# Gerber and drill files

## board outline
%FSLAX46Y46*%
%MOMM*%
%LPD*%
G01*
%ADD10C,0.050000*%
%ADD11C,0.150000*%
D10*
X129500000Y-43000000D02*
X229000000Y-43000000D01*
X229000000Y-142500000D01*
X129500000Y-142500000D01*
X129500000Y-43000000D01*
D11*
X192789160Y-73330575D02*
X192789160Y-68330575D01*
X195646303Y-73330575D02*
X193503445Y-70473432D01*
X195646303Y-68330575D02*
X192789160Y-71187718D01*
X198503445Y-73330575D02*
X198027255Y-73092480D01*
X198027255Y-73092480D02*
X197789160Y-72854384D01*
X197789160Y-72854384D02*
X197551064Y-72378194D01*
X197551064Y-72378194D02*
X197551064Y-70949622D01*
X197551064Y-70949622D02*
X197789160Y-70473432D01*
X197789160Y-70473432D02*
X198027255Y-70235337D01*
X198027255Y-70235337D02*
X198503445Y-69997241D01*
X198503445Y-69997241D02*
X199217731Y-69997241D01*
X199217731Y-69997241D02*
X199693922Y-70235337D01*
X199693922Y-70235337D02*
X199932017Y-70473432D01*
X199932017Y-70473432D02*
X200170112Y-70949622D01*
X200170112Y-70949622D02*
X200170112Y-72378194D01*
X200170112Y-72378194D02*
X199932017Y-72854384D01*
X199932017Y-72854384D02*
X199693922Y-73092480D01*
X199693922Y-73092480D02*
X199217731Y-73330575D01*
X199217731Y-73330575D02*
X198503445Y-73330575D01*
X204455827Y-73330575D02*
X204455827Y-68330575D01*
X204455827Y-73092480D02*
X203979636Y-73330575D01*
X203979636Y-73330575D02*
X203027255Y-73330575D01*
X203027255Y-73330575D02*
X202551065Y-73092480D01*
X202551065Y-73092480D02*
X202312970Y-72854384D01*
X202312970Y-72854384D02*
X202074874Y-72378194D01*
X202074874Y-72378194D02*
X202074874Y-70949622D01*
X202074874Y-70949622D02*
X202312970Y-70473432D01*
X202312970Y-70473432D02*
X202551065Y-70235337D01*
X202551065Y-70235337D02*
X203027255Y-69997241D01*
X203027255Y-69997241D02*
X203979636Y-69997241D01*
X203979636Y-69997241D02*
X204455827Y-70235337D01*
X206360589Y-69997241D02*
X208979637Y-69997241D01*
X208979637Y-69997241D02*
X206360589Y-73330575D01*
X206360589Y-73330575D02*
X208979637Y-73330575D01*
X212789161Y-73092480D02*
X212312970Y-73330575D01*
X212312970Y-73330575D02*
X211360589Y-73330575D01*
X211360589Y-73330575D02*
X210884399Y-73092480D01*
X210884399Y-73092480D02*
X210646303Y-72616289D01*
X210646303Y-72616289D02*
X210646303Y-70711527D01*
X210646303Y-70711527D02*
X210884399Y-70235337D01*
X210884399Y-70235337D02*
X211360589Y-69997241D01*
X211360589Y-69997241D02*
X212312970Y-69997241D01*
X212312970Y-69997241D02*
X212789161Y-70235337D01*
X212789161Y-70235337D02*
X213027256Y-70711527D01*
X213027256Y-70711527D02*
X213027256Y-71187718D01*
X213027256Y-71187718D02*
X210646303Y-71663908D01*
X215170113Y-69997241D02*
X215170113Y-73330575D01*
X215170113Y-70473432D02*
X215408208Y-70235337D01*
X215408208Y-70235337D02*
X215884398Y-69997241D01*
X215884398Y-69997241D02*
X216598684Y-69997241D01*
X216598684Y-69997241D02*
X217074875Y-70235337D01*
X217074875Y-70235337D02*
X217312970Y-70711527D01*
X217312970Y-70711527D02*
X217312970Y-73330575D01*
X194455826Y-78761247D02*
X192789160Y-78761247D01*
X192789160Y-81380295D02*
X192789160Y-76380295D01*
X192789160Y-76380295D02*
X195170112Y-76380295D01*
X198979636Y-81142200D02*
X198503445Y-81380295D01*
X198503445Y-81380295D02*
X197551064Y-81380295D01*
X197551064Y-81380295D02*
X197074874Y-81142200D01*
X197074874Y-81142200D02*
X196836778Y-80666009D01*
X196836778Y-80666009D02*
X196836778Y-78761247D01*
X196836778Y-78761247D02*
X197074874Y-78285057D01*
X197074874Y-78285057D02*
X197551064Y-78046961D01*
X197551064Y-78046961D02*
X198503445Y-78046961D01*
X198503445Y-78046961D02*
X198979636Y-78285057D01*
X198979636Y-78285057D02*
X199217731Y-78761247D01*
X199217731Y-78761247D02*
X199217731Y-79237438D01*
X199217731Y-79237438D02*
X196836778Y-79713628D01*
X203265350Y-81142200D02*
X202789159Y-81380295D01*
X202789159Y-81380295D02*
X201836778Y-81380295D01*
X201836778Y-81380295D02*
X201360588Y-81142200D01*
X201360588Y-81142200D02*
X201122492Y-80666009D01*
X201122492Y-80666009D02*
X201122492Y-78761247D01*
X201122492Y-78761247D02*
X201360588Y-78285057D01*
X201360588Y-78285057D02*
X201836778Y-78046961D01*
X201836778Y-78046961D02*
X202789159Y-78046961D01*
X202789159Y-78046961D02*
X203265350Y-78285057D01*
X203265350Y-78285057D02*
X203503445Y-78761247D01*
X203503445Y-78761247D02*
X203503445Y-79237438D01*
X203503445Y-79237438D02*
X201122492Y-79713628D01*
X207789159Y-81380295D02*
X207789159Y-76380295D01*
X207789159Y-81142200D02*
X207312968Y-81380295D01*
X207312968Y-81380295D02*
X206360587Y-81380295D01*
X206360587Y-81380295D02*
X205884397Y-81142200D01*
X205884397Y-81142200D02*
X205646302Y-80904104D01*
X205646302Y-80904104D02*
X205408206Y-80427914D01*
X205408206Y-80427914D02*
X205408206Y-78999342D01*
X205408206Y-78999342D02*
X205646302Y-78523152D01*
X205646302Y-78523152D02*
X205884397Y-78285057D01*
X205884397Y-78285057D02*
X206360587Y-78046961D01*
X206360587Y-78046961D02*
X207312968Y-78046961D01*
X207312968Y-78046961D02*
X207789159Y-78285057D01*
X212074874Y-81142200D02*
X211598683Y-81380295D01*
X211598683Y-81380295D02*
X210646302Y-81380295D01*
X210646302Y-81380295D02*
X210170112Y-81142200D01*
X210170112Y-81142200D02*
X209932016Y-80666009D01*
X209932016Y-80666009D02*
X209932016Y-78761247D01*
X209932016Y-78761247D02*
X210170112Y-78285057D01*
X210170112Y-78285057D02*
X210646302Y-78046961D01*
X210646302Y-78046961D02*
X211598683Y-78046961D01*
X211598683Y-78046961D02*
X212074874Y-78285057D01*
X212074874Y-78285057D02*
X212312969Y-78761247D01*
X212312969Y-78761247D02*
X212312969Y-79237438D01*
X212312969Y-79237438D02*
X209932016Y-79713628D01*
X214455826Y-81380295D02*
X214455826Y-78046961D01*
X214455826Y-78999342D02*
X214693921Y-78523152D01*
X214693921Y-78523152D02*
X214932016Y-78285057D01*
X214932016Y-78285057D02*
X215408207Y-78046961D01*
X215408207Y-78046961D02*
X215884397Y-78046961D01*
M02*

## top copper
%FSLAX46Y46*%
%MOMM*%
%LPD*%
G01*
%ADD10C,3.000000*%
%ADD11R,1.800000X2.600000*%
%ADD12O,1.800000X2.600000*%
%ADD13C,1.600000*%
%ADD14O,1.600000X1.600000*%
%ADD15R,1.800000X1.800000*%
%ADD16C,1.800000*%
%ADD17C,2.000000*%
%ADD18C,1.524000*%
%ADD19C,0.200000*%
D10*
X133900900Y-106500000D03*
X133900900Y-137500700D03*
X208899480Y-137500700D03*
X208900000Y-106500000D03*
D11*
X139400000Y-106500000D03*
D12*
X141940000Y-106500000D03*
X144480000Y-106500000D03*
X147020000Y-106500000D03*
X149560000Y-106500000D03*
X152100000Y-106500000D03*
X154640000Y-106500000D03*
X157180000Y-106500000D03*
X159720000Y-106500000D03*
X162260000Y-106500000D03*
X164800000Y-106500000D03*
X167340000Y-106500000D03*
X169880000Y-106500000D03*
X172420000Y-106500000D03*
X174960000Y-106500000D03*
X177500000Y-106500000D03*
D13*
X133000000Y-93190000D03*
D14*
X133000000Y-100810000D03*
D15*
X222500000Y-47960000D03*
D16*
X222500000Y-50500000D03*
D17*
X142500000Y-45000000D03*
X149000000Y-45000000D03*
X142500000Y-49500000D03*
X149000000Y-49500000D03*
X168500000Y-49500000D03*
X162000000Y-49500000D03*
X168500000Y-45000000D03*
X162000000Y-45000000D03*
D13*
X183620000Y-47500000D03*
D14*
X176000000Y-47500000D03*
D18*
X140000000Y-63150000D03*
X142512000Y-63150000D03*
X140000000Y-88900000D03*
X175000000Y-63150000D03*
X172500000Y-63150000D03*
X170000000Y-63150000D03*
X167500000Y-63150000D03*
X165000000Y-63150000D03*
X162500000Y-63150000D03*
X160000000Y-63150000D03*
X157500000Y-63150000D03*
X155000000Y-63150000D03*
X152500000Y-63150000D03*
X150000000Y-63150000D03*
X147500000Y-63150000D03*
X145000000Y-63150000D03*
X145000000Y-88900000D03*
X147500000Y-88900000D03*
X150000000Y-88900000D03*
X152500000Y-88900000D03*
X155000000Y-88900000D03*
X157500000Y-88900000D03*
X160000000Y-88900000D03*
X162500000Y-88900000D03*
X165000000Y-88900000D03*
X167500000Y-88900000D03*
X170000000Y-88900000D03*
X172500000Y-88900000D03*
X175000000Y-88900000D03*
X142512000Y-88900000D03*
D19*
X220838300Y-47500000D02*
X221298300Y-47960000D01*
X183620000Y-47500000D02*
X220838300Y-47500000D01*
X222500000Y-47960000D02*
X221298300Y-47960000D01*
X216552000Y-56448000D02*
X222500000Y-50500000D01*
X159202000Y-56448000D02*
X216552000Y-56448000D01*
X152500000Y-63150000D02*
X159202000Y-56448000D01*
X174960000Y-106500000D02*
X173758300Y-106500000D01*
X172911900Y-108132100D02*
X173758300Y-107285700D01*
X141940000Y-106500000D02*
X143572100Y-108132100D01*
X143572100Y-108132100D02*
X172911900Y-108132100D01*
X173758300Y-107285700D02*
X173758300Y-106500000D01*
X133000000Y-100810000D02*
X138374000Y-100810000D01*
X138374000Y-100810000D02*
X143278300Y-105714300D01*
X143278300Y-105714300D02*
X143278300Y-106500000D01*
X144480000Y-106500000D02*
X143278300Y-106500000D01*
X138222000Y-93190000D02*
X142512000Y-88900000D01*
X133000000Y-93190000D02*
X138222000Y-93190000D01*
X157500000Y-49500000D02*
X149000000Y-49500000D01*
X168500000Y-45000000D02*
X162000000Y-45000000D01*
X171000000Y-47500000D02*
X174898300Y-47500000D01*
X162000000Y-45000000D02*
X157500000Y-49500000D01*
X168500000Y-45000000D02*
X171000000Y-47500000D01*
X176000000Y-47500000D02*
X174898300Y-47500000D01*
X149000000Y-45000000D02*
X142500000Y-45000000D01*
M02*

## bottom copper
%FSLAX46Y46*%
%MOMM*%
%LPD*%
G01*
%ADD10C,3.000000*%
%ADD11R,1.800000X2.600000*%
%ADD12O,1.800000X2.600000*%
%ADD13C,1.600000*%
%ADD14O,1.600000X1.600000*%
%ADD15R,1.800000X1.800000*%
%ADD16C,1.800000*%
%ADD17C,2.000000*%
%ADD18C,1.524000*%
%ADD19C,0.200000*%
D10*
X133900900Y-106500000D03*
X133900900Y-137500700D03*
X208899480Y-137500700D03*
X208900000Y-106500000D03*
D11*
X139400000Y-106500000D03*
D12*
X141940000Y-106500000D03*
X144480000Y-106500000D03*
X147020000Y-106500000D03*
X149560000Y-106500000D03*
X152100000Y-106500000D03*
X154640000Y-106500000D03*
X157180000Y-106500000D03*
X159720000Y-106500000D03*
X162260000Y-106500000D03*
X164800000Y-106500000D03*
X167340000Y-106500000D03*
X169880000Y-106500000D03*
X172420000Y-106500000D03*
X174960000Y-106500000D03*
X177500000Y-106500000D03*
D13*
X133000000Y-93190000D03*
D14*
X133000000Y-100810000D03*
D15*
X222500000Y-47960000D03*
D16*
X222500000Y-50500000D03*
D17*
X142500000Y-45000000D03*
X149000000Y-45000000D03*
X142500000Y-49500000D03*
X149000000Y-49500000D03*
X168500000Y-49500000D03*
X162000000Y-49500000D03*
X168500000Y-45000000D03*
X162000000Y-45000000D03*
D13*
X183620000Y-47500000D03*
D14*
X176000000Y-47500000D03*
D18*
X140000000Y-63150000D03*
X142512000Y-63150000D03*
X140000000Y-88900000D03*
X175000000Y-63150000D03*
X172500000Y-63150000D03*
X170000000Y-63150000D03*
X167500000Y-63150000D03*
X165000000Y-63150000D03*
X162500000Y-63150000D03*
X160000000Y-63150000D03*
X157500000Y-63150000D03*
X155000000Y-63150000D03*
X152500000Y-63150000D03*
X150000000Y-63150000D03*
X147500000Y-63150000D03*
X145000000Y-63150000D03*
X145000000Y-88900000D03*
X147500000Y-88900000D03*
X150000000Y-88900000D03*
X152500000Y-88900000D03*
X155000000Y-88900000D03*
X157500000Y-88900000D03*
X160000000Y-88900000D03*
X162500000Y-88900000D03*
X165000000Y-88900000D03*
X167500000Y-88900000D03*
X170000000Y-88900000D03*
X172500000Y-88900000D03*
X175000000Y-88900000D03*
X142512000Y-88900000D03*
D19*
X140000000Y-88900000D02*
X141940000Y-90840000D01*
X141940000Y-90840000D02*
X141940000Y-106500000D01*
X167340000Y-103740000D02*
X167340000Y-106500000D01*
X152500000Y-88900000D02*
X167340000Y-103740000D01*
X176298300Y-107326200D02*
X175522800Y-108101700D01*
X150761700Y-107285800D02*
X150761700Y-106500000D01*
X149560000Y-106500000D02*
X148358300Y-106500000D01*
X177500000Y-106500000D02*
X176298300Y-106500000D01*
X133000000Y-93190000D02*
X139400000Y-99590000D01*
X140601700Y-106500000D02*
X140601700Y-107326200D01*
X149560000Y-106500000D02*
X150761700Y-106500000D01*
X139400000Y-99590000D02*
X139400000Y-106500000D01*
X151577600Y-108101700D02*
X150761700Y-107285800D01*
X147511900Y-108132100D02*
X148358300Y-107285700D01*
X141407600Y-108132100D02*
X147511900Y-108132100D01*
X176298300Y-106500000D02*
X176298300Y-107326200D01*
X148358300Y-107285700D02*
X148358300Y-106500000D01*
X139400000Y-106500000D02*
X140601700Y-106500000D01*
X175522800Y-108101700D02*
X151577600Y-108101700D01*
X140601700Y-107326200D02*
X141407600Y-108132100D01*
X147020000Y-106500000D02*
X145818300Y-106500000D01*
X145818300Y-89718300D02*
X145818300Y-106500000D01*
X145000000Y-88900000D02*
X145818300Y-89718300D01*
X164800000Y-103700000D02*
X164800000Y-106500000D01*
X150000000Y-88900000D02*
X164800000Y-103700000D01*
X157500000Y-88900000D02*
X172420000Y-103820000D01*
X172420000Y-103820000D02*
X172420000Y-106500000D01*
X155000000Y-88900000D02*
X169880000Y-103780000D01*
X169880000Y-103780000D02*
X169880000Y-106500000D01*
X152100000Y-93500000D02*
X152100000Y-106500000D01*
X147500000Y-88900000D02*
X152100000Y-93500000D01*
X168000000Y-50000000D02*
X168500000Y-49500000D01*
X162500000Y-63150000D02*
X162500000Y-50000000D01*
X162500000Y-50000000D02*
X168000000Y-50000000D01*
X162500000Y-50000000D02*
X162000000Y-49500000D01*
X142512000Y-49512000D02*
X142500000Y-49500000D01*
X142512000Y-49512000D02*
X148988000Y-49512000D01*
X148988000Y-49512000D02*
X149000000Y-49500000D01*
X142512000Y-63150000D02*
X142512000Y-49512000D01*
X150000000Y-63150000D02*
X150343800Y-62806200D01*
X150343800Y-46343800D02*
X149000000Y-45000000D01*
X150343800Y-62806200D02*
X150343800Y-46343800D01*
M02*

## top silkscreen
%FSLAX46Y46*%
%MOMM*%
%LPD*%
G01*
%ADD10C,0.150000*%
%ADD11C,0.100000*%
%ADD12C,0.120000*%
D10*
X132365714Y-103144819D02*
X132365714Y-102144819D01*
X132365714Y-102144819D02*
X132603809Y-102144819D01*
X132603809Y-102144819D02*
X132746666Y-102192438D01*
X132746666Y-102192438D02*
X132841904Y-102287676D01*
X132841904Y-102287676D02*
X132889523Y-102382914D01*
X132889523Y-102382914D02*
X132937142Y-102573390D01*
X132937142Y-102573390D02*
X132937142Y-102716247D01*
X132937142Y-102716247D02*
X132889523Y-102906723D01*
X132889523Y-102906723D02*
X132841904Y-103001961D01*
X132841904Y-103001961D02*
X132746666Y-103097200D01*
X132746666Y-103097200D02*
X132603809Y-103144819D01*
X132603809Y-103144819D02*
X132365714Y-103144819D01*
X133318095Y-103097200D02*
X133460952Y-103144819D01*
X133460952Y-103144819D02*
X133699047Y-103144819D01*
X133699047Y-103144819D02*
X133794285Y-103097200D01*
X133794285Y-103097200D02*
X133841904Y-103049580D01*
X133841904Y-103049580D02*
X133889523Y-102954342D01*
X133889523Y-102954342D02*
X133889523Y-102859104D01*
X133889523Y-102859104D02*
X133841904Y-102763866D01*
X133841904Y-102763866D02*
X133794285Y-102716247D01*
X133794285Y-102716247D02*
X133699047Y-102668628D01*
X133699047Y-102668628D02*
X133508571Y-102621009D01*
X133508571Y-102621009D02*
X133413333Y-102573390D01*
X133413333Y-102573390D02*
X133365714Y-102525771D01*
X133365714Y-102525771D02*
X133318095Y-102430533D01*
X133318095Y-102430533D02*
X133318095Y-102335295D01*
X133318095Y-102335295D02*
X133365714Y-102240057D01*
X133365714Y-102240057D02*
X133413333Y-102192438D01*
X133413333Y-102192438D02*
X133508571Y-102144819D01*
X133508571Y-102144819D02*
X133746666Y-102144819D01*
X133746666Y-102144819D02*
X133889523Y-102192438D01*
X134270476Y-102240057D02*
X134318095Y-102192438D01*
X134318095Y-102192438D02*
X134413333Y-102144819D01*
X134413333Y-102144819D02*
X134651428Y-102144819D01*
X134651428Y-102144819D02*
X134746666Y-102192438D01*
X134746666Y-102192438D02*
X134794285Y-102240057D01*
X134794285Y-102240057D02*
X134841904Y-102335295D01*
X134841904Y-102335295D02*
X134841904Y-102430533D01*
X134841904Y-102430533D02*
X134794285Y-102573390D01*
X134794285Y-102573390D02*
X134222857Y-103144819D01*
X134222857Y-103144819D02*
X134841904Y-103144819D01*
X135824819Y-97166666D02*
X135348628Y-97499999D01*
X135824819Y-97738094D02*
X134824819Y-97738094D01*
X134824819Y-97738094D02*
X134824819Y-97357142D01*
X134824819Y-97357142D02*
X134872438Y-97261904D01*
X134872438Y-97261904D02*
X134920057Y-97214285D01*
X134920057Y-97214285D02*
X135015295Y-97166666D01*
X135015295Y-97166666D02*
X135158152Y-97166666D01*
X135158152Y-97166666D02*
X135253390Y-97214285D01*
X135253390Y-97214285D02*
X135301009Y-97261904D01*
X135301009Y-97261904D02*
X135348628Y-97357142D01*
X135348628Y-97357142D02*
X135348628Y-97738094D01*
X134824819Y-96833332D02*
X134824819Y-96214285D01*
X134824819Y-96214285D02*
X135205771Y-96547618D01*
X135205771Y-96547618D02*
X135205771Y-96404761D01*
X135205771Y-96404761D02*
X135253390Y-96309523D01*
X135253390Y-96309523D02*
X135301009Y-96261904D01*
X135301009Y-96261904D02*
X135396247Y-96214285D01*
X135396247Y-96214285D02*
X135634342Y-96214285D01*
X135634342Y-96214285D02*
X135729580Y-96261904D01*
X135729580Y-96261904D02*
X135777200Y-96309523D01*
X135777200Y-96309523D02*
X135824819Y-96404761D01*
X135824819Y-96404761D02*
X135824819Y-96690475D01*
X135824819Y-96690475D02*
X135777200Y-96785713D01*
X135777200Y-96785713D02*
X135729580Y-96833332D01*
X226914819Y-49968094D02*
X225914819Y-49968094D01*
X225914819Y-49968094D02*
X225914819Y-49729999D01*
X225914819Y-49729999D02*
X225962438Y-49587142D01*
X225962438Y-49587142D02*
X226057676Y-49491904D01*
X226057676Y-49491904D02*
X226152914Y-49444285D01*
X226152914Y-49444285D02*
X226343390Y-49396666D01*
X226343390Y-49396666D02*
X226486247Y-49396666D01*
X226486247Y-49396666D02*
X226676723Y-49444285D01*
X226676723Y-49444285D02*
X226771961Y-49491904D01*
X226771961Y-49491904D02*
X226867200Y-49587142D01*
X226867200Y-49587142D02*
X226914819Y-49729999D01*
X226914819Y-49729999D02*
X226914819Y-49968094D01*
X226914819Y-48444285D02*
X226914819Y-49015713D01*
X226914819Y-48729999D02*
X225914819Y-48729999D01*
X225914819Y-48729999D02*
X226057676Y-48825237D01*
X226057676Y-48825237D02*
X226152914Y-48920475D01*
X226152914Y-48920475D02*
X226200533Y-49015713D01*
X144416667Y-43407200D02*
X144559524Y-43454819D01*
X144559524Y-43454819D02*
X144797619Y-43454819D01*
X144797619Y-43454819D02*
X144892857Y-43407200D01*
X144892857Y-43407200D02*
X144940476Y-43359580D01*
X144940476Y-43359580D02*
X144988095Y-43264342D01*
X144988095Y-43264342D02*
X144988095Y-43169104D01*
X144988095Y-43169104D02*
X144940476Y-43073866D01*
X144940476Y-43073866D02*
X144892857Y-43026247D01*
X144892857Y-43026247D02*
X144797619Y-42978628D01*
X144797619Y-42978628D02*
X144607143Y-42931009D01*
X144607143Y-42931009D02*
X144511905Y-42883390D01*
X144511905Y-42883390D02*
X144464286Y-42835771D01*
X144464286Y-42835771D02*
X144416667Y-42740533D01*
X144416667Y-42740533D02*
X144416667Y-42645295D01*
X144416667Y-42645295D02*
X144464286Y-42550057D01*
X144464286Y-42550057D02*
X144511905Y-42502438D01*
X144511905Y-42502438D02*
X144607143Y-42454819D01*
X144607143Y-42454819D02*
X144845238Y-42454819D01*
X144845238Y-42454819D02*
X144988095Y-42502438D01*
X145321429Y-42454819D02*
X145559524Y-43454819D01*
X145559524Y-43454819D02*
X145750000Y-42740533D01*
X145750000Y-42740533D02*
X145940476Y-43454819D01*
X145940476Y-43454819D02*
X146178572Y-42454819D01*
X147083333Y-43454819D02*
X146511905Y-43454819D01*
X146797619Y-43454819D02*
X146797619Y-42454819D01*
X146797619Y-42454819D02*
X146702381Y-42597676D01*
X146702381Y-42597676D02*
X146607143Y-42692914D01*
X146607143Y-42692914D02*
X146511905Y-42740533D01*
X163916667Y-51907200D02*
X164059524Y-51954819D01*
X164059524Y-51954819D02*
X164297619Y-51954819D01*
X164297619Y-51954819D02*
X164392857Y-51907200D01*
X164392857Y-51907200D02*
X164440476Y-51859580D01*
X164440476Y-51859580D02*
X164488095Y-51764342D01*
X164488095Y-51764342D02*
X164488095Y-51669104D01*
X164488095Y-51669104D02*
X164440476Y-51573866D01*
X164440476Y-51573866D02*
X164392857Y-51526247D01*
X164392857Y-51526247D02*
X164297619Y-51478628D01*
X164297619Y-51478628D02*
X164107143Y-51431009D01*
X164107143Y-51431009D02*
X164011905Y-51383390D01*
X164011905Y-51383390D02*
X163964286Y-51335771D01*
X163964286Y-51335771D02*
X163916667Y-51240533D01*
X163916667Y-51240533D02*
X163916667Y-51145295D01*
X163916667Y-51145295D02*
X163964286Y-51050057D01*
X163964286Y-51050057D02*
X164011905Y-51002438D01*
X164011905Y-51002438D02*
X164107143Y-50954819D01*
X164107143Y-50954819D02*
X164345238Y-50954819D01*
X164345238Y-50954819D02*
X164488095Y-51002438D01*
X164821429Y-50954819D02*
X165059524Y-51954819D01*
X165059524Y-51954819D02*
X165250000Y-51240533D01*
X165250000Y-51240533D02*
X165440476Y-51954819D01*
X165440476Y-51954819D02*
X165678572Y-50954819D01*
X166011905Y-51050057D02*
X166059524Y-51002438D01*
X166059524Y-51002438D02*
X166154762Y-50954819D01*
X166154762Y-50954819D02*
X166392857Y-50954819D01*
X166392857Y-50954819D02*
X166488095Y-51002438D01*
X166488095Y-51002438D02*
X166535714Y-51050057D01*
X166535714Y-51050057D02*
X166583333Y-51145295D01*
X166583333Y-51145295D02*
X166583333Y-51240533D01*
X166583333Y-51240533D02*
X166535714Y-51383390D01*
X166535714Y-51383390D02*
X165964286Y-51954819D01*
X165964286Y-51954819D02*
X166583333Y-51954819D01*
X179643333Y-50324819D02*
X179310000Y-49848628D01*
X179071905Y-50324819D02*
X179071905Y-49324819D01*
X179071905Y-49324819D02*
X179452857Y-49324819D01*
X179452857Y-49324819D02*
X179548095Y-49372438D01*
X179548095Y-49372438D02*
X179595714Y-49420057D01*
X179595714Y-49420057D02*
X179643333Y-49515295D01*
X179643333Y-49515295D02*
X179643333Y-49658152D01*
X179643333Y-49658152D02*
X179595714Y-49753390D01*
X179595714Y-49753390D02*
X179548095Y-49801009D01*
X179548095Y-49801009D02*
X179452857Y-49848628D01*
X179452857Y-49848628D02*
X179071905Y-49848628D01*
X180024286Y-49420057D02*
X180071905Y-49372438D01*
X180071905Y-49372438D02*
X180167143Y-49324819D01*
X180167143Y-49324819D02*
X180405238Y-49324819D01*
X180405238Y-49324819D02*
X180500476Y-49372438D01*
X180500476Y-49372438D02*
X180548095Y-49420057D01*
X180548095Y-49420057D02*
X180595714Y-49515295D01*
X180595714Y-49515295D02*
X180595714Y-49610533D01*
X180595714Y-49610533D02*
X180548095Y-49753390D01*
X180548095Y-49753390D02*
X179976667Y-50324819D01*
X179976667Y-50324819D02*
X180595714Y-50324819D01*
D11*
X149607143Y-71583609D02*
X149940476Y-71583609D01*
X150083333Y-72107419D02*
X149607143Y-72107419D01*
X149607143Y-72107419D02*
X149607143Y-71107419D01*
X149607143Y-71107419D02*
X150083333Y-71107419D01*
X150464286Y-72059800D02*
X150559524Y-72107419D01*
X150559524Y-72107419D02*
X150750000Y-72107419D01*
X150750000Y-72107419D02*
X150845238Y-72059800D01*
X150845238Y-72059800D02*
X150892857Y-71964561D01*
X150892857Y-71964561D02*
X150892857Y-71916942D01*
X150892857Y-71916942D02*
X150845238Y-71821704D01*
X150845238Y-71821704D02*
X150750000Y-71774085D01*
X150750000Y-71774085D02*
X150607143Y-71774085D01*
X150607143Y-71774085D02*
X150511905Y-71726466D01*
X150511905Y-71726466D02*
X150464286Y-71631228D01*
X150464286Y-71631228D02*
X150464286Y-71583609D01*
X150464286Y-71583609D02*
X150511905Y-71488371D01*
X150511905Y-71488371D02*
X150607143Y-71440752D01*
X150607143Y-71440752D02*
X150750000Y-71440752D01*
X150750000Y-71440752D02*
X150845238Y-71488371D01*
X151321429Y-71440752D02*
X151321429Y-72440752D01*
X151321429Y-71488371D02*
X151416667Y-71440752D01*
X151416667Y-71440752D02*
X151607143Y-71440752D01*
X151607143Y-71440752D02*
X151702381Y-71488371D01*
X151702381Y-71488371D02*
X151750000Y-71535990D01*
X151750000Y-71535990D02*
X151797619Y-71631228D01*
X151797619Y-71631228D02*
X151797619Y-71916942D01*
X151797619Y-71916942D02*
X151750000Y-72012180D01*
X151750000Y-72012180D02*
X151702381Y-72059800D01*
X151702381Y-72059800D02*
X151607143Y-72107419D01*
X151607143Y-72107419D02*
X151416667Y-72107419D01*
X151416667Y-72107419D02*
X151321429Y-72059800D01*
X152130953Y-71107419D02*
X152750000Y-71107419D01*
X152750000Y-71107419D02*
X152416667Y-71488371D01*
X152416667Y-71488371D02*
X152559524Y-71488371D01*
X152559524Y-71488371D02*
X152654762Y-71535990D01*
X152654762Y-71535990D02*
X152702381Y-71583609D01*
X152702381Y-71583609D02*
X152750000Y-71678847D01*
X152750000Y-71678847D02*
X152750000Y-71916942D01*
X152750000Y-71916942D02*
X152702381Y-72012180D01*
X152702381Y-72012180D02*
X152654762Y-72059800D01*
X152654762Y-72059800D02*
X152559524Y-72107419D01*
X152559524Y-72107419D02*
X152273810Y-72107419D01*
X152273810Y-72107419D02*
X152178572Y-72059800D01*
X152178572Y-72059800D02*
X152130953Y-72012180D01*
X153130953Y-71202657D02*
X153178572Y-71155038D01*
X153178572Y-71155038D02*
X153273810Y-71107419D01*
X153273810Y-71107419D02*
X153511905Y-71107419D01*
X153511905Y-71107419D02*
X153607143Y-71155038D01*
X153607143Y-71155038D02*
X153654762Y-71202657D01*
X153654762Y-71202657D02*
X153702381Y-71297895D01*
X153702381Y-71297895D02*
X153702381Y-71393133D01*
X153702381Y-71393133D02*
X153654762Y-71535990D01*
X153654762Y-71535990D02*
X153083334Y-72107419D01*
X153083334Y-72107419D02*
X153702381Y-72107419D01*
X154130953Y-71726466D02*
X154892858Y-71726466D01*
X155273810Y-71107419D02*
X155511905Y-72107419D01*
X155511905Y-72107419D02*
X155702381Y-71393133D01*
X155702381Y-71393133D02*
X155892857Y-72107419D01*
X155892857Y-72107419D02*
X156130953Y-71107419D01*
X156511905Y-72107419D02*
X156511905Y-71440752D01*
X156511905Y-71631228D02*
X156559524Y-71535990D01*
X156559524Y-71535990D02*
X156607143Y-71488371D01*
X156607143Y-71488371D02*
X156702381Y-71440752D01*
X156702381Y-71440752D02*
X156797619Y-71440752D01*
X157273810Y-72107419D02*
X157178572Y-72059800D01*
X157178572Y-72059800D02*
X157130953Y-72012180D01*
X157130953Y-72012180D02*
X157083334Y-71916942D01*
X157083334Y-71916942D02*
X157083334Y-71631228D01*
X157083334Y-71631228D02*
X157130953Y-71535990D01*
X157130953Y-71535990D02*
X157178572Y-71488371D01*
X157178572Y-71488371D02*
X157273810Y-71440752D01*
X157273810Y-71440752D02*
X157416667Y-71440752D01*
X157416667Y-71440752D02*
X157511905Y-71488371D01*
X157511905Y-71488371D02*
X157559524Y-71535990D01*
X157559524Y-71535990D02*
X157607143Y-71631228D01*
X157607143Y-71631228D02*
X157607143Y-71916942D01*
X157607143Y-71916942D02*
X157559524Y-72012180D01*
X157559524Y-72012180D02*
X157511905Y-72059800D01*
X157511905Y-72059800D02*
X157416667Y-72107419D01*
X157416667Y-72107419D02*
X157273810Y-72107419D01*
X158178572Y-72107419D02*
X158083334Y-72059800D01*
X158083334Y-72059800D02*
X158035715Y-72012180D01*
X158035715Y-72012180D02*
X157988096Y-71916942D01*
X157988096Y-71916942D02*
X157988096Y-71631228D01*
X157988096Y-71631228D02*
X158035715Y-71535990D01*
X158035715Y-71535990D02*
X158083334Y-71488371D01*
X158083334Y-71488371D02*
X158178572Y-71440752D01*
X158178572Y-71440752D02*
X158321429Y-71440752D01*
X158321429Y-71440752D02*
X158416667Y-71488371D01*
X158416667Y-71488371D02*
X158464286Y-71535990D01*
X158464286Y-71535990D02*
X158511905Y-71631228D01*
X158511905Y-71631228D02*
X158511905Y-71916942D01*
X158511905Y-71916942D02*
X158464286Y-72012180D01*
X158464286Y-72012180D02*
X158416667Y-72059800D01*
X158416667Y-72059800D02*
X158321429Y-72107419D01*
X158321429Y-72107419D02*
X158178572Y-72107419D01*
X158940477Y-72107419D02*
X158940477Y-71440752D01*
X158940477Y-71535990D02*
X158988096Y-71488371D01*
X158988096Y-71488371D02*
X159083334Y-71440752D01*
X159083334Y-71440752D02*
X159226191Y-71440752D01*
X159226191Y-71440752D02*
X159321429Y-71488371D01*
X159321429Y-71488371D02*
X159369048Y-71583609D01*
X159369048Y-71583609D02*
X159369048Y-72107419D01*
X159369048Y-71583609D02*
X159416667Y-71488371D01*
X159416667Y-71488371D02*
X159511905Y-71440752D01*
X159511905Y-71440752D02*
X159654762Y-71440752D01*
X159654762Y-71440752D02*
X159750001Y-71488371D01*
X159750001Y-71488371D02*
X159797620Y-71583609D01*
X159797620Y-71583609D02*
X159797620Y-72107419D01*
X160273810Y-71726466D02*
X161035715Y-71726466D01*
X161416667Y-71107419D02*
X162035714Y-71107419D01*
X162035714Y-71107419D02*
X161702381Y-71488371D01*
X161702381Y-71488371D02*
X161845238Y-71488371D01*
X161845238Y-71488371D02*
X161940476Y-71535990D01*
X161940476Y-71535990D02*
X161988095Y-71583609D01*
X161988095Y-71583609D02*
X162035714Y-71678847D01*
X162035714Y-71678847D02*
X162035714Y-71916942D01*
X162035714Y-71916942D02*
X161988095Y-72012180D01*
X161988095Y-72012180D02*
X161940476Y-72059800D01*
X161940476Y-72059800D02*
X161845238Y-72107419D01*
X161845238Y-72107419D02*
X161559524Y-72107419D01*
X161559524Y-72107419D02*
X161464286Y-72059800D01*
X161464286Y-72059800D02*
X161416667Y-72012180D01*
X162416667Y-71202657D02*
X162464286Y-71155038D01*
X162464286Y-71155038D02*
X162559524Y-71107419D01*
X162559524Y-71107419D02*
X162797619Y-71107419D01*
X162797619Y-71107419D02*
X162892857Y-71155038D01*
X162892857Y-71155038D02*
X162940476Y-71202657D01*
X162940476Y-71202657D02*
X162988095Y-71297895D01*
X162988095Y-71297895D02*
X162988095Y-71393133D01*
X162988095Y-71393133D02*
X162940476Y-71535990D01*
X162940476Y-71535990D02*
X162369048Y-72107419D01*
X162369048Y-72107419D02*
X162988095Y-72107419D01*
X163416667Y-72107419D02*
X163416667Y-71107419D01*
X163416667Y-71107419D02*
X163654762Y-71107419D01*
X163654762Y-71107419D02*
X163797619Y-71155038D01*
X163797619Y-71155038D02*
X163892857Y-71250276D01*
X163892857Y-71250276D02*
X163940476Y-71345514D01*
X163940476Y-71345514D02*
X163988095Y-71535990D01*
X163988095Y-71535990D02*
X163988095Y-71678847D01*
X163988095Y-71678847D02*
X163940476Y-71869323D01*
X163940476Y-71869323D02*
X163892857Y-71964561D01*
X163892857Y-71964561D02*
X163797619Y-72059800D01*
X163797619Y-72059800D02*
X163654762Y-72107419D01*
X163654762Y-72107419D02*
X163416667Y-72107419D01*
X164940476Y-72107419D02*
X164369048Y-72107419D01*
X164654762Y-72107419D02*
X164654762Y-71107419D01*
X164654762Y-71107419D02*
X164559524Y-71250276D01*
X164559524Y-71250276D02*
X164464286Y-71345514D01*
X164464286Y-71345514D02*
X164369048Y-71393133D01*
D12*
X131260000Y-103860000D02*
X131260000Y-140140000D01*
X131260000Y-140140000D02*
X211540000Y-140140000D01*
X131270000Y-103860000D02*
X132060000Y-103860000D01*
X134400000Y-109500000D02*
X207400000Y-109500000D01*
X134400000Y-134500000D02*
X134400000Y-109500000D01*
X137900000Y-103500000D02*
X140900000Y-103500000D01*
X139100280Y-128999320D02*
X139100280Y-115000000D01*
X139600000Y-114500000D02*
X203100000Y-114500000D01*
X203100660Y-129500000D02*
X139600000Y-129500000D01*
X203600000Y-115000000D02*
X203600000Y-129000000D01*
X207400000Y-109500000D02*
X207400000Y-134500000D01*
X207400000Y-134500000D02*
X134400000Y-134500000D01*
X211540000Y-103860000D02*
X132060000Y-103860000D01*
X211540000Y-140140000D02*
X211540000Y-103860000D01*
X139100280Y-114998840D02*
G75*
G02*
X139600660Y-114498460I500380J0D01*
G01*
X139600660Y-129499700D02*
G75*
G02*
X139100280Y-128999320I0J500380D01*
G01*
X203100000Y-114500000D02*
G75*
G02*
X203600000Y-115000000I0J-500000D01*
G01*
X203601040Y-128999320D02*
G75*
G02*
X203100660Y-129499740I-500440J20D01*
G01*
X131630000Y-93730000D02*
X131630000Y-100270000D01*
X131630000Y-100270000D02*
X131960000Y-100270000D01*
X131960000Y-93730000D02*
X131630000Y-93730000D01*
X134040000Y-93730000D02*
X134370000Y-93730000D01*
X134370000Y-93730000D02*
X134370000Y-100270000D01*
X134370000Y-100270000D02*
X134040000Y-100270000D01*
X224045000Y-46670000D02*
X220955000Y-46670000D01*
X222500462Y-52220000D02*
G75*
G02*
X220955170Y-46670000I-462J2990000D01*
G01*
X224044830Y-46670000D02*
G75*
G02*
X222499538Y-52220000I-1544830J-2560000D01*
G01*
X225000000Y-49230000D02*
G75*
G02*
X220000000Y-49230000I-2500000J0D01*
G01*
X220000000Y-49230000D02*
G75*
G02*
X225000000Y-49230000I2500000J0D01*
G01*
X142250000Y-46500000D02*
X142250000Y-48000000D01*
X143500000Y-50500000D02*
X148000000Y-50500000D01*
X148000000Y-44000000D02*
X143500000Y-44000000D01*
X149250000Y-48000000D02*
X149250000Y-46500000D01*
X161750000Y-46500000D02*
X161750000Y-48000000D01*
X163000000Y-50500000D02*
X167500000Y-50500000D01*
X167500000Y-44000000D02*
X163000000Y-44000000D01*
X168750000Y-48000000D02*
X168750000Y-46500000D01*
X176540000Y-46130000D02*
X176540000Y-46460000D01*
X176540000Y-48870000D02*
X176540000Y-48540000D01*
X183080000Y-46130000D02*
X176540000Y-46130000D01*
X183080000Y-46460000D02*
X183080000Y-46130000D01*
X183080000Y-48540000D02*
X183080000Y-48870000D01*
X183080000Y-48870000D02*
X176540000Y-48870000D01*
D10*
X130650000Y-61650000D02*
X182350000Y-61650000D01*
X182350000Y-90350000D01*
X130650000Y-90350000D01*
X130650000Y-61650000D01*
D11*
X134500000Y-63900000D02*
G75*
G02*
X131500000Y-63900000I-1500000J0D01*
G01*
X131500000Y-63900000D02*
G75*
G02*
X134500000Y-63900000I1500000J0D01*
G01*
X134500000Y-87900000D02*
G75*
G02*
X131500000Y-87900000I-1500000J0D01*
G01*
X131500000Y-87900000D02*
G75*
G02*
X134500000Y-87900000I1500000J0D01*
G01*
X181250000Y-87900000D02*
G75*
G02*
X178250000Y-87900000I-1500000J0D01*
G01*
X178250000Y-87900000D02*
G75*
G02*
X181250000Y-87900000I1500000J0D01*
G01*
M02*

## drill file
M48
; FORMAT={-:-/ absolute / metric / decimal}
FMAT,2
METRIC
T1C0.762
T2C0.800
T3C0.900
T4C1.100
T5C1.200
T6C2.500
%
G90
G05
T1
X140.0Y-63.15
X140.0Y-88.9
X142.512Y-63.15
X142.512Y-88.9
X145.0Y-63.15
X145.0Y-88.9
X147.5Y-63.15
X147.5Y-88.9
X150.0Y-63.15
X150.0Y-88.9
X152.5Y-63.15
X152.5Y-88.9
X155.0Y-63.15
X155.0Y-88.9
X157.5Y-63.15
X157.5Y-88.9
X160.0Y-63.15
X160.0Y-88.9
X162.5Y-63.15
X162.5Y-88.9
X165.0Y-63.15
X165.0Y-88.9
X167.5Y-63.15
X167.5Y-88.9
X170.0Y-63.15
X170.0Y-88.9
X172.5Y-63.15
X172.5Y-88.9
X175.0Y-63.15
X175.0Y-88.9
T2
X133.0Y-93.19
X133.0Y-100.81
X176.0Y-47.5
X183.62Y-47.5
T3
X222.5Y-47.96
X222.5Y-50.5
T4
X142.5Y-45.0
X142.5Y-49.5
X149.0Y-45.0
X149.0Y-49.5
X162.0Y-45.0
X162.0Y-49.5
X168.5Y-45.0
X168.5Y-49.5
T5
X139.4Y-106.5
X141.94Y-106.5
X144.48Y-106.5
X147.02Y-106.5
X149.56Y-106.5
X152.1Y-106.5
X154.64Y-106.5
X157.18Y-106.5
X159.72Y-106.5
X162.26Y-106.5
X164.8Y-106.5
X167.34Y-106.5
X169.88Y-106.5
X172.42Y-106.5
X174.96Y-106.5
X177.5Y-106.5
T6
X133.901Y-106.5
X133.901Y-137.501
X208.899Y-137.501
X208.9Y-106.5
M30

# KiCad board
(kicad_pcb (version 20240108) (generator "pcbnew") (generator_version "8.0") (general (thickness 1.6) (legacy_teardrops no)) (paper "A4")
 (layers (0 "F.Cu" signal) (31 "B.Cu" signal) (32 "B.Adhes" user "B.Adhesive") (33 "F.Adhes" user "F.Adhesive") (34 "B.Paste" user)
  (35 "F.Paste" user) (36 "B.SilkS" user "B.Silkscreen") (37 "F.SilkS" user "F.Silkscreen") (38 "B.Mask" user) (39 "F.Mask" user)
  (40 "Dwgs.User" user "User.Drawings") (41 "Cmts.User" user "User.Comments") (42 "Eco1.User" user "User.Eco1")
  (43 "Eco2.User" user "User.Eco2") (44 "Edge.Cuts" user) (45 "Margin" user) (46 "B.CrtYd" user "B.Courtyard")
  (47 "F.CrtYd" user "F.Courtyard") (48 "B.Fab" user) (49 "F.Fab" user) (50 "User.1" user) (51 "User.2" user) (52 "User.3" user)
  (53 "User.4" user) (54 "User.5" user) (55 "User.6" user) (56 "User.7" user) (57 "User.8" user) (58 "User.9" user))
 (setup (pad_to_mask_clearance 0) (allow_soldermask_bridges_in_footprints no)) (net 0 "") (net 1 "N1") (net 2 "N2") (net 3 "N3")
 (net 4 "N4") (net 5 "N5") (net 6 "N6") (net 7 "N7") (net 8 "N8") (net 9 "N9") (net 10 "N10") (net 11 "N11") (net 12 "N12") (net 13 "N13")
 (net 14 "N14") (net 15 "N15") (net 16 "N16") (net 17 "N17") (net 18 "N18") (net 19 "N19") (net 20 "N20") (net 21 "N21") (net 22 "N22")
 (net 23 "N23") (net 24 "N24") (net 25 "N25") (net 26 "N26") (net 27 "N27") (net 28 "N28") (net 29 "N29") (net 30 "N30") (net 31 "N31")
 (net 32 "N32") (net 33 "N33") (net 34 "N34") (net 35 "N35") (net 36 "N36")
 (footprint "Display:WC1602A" (layer "F.Cu") (at 139.4 106.5)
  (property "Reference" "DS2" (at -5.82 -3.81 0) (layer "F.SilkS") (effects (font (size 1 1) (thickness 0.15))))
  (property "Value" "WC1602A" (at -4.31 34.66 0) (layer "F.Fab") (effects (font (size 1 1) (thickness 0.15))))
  (fp_line (start -8.14 -2.64) (end -8.14 33.64) (stroke (width 0.12) (type solid)) (layer "F.SilkS"))
  (fp_line (start -8.14 33.64) (end 72.14 33.64) (stroke (width 0.12) (type solid)) (layer "F.SilkS"))
  (fp_line (start -8.13 -2.64) (end -7.34 -2.64) (stroke (width 0.12) (type solid)) (layer "F.SilkS"))
  (fp_line (start -5 3) (end 68 3) (stroke (width 0.12) (type solid)) (layer "F.SilkS"))
  (fp_line (start -5 28) (end -5 3) (stroke (width 0.12) (type solid)) (layer "F.SilkS"))
  (fp_line (start -1.5 -3) (end 1.5 -3) (stroke (width 0.12) (type solid)) (layer "F.SilkS"))
  (fp_line (start -0.29972 22.49932) (end -0.29972 8.5) (stroke (width 0.12) (type solid)) (layer "F.SilkS"))
  (fp_line (start 0.2 8) (end 63.7 8) (stroke (width 0.12) (type solid)) (layer "F.SilkS"))
  (fp_line (start 63.70066 23) (end 0.2 23) (stroke (width 0.12) (type solid)) (layer "F.SilkS"))
  (fp_line (start 64.2 8.5) (end 64.2 22.5) (stroke (width 0.12) (type solid)) (layer "F.SilkS"))
  (fp_line (start 68 3) (end 68 28) (stroke (width 0.12) (type solid)) (layer "F.SilkS"))
  (fp_line (start 68 28) (end -5 28) (stroke (width 0.12) (type solid)) (layer "F.SilkS"))
  (fp_line (start 72.14 -2.64) (end -7.34 -2.64) (stroke (width 0.12) (type solid)) (layer "F.SilkS"))
  (fp_line (start 72.14 33.64) (end 72.14 -2.64) (stroke (width 0.12) (type solid)) (layer "F.SilkS"))
  (fp_arc (start -0.29972 8.49884) (mid -0.153162 8.145018) (end 0.20066 7.99846) (stroke (width 0.12) (type solid)) (layer "F.SilkS"))
  (fp_arc (start 0.20066 22.9997) (mid -0.153162 22.853142) (end -0.29972 22.49932) (stroke (width 0.12) (type solid)) (layer "F.SilkS"))
  (fp_arc (start 63.7 8) (mid 64.053553 8.146447) (end 64.2 8.5) (stroke (width 0.12) (type solid)) (layer "F.SilkS"))
  (fp_arc (start 64.20104 22.49932) (mid 64.054473 22.853115) (end 63.70066 22.9997) (stroke (width 0.12) (type solid)) (layer "F.SilkS"))
  (pad "" thru_hole circle (at -5.4991 0) (size 3 3) (drill 2.5) (layers "*.Cu" "*.Mask") (remove_unused_layers no))
  (pad "" thru_hole circle (at -5.4991 31.0007) (size 3 3) (drill 2.5) (layers "*.Cu" "*.Mask") (remove_unused_layers no))
  (pad "" thru_hole circle (at 69.49948 31.0007) (size 3 3) (drill 2.5) (layers "*.Cu" "*.Mask") (remove_unused_layers no))
  (pad "" thru_hole circle (at 69.5 0) (size 3 3) (drill 2.5) (layers "*.Cu" "*.Mask") (remove_unused_layers no))
  (pad "1" thru_hole rect (at 0 0) (size 1.8 2.6) (drill 1.2) (layers "*.Cu" "*.Mask") (remove_unused_layers no) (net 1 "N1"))
  (pad "2" thru_hole oval (at 2.54 0) (size 1.8 2.6) (drill 1.2) (layers "*.Cu" "*.Mask") (remove_unused_layers no) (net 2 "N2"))
  (pad "3" thru_hole oval (at 5.08 0) (size 1.8 2.6) (drill 1.2) (layers "*.Cu" "*.Mask") (remove_unused_layers no) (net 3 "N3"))
  (pad "4" thru_hole oval (at 7.62 0) (size 1.8 2.6) (drill 1.2) (layers "*.Cu" "*.Mask") (remove_unused_layers no) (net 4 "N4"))
  (pad "5" thru_hole oval (at 10.16 0) (size 1.8 2.6) (drill 1.2) (layers "*.Cu" "*.Mask") (remove_unused_layers no) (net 1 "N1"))
  (pad "6" thru_hole oval (at 12.7 0) (size 1.8 2.6) (drill 1.2) (layers "*.Cu" "*.Mask") (remove_unused_layers no) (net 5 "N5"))
  (pad "7" thru_hole oval (at 15.24 0) (size 1.8 2.6) (drill 1.2) (layers "*.Cu" "*.Mask") (remove_unused_layers no) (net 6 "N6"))
  (pad "8" thru_hole oval (at 17.78 0) (size 1.8 2.6) (drill 1.2) (layers "*.Cu" "*.Mask") (remove_unused_layers no) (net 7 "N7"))
  (pad "9" thru_hole oval (at 20.32 0) (size 1.8 2.6) (drill 1.2) (layers "*.Cu" "*.Mask") (remove_unused_layers no) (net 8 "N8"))
  (pad "10" thru_hole oval (at 22.86 0) (size 1.8 2.6) (drill 1.2) (layers "*.Cu" "*.Mask") (remove_unused_layers no) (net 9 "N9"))
  (pad "11" thru_hole oval (at 25.4 0) (size 1.8 2.6) (drill 1.2) (layers "*.Cu" "*.Mask") (remove_unused_layers no) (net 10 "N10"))
  (pad "12" thru_hole oval (at 27.94 0) (size 1.8 2.6) (drill 1.2) (layers "*.Cu" "*.Mask") (remove_unused_layers no) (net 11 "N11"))
  (pad "13" thru_hole oval (at 30.48 0) (size 1.8 2.6) (drill 1.2) (layers "*.Cu" "*.Mask") (remove_unused_layers no) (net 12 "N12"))
  (pad "14" thru_hole oval (at 33.02 0) (size 1.8 2.6) (drill 1.2) (layers "*.Cu" "*.Mask") (remove_unused_layers no) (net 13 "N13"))
  (pad "15" thru_hole oval (at 35.56 0) (size 1.8 2.6) (drill 1.2) (layers "*.Cu" "*.Mask") (remove_unused_layers no) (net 2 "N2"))
  (pad "16" thru_hole oval (at 38.1 0) (size 1.8 2.6) (drill 1.2) (layers "*.Cu" "*.Mask") (remove_unused_layers no) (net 1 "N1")))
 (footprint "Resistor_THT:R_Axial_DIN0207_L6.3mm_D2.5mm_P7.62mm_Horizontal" (layer "F.Cu") (at 133 93.19 -90)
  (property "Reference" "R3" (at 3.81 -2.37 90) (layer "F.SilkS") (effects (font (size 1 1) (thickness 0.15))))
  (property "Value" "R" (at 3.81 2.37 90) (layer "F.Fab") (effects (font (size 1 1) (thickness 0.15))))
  (fp_line (start 0.54 1.37) (end 7.08 1.37) (stroke (width 0.12) (type solid)) (layer "F.SilkS"))
  (fp_line (start 7.08 1.37) (end 7.08 1.04) (stroke (width 0.12) (type solid)) (layer "F.SilkS"))
  (fp_line (start 0.54 1.04) (end 0.54 1.37) (stroke (width 0.12) (type solid)) (layer "F.SilkS"))
  (fp_line (start 0.54 -1.04) (end 0.54 -1.37) (stroke (width 0.12) (type solid)) (layer "F.SilkS"))
  (fp_line (start 0.54 -1.37) (end 7.08 -1.37) (stroke (width 0.12) (type solid)) (layer "F.SilkS"))
  (fp_line (start 7.08 -1.37) (end 7.08 -1.04) (stroke (width 0.12) (type solid)) (layer "F.SilkS"))
  (pad "1" thru_hole circle (at 0 0 270) (size 1.6 1.6) (drill 0.8) (layers "*.Cu" "*.Mask") (remove_unused_layers no) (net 1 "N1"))
  (pad "2" thru_hole oval (at 7.62 0 270) (size 1.6 1.6) (drill 0.8) (layers "*.Cu" "*.Mask") (remove_unused_layers no) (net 3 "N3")))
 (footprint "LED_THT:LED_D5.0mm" (layer "F.Cu") (at 222.5 47.96 -90)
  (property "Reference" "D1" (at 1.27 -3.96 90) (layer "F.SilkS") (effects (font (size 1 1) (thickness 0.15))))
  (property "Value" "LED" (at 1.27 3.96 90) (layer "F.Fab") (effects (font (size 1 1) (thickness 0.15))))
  (fp_line (start -1.29 -1.545) (end -1.29 1.545) (stroke (width 0.12) (type solid)) (layer "F.SilkS"))
  (fp_arc (start 4.26 -0.000462) (mid 2.072002 2.880433) (end -1.29 1.54483) (stroke (width 0.12) (type solid)) (layer "F.SilkS"))
  (fp_arc (start -1.29 -1.54483) (mid 2.072002 -2.880433) (end 4.26 0.000462) (stroke (width 0.12) (type solid)) (layer "F.SilkS"))
  (fp_circle (center 1.27 0) (end 3.77 0) (stroke (width 0.12) (type solid)) (fill none) (layer "F.SilkS"))
  (pad "1" thru_hole rect (at 0 0 270) (size 1.8 1.8) (drill 0.9) (layers "*.Cu" "*.Mask") (remove_unused_layers no) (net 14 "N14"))
  (pad "2" thru_hole circle (at 2.54 0 270) (size 1.8 1.8) (drill 0.9) (layers "*.Cu" "*.Mask") (remove_unused_layers no) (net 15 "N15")))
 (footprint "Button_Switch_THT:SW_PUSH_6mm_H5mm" (layer "F.Cu") (at 142.5 45)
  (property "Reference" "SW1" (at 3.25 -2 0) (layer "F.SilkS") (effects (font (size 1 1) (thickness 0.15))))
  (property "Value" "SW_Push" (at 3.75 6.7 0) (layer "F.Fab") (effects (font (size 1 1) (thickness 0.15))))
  (fp_line (start -0.25 1.5) (end -0.25 3) (stroke (width 0.12) (type solid)) (layer "F.SilkS"))
  (fp_line (start 1 5.5) (end 5.5 5.5) (stroke (width 0.12) (type solid)) (layer "F.SilkS"))
  (fp_line (start 5.5 -1) (end 1 -1) (stroke (width 0.12) (type solid)) (layer "F.SilkS"))
  (fp_line (start 6.75 3) (end 6.75 1.5) (stroke (width 0.12) (type solid)) (layer "F.SilkS"))
  (pad "1" thru_hole circle (at 0 0 90) (size 2 2) (drill 1.1) (layers "*.Cu" "*.Mask") (remove_unused_layers no) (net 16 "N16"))
  (pad "1" thru_hole circle (at 6.5 0 90) (size 2 2) (drill 1.1) (layers "*.Cu" "*.Mask") (remove_unused_layers no) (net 16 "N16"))
  (pad "2" thru_hole circle (at 0 4.5 90) (size 2 2) (drill 1.1) (layers "*.Cu" "*.Mask") (remove_unused_layers no) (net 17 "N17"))
  (pad "2" thru_hole circle (at 6.5 4.5 90) (size 2 2) (drill 1.1) (layers "*.Cu" "*.Mask") (remove_unused_layers no) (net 17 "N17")))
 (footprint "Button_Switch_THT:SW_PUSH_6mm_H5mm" (layer "F.Cu") (at 168.5 49.5 180)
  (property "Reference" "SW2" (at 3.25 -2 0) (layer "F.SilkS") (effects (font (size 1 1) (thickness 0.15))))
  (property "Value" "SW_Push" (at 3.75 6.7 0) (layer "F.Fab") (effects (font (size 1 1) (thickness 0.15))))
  (fp_line (start 6.75 3) (end 6.75 1.5) (stroke (width 0.12) (type solid)) (layer "F.SilkS"))
  (fp_line (start 5.5 -1) (end 1 -1) (stroke (width 0.12) (type solid)) (layer "F.SilkS"))
  (fp_line (start 1 5.5) (end 5.5 5.5) (stroke (width 0.12) (type solid)) (layer "F.SilkS"))
  (fp_line (start -0.25 1.5) (end -0.25 3) (stroke (width 0.12) (type solid)) (layer "F.SilkS"))
  (pad "1" thru_hole circle (at 0 0 270) (size 2 2) (drill 1.1) (layers "*.Cu" "*.Mask") (remove_unused_layers no) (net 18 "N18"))
  (pad "1" thru_hole circle (at 6.5 0 270) (size 2 2) (drill 1.1) (layers "*.Cu" "*.Mask") (remove_unused_layers no) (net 18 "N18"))
  (pad "2" thru_hole circle (at 0 4.5 270) (size 2 2) (drill 1.1) (layers "*.Cu" "*.Mask") (remove_unused_layers no) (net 17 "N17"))
  (pad "2" thru_hole circle (at 6.5 4.5 270) (size 2 2) (drill 1.1) (layers "*.Cu" "*.Mask") (remove_unused_layers no) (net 17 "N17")))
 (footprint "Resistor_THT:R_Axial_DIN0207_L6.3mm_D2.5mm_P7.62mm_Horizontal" (layer "F.Cu") (at 183.62 47.5 180)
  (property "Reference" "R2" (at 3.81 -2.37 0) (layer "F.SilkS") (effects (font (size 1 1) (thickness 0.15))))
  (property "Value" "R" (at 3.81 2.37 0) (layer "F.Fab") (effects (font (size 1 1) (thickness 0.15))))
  (fp_line (start 7.08 1.37) (end 7.08 1.04) (stroke (width 0.12) (type solid)) (layer "F.SilkS"))
  (fp_line (start 7.08 -1.37) (end 7.08 -1.04) (stroke (width 0.12) (type solid)) (layer "F.SilkS"))
  (fp_line (start 0.54 1.37) (end 7.08 1.37) (stroke (width 0.12) (type solid)) (layer "F.SilkS"))
  (fp_line (start 0.54 1.04) (end 0.54 1.37) (stroke (width 0.12) (type solid)) (layer "F.SilkS"))
  (fp_line (start 0.54 -1.04) (end 0.54 -1.37) (stroke (width 0.12) (type solid)) (layer "F.SilkS"))
  (fp_line (start 0.54 -1.37) (end 7.08 -1.37) (stroke (width 0.12) (type solid)) (layer "F.SilkS"))
  (pad "1" thru_hole circle (at 0 0 180) (size 1.6 1.6) (drill 0.8) (layers "*.Cu" "*.Mask") (remove_unused_layers no) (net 14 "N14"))
  (pad "2" thru_hole oval (at 7.62 0 180) (size 1.6 1.6) (drill 0.8) (layers "*.Cu" "*.Mask") (remove_unused_layers no) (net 17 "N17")))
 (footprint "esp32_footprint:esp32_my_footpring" (layer "F.Cu") (at 157.25 72.15)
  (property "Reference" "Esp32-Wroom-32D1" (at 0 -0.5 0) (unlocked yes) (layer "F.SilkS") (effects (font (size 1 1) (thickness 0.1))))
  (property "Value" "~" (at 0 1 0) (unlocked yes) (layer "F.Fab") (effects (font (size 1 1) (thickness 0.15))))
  (fp_rect (start -26.6 -10.5) (end 25.1 18.2) (stroke (width 0.15) (type default)) (fill none) (layer "F.SilkS"))
  (fp_circle (center -24.25 -8.25) (end -22.75 -8.25) (stroke (width 0.1) (type default)) (fill none) (layer "F.SilkS"))
  (fp_circle (center -24.25 15.75) (end -22.75 15.75) (stroke (width 0.1) (type default)) (fill none) (layer "F.SilkS"))
  (fp_circle (center 22.5 15.75) (end 24 15.75) (stroke (width 0.1) (type default)) (fill none) (layer "F.SilkS"))
  (pad "0" thru_hole circle (at -17.25 -9) (size 1.524 1.524) (drill 0.762) (layers "*.Cu" "*.Mask") (remove_unused_layers no)
   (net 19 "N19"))
  (pad "1" thru_hole circle (at -14.738 -9) (size 1.524 1.524) (drill 0.762) (layers "*.Cu" "*.Mask") (remove_unused_layers no)
   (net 17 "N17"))
  (pad "2" thru_hole circle (at -17.25 16.75) (size 1.524 1.524) (drill 0.762) (layers "*.Cu" "*.Mask") (remove_unused_layers no)
   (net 2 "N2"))
  (pad "3" thru_hole circle (at 17.75 -9) (size 1.524 1.524) (drill 0.762) (layers "*.Cu" "*.Mask") (remove_unused_layers no) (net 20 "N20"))
  (pad "4" thru_hole circle (at 15.25 -9) (size 1.524 1.524) (drill 0.762) (layers "*.Cu" "*.Mask") (remove_unused_layers no) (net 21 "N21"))
  (pad "5" thru_hole circle (at 12.75 -9) (size 1.524 1.524) (drill 0.762) (layers "*.Cu" "*.Mask") (remove_unused_layers no) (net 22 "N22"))
  (pad "6" thru_hole circle (at 10.25 -9) (size 1.524 1.524) (drill 0.762) (layers "*.Cu" "*.Mask") (remove_unused_layers no) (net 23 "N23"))
  (pad "7" thru_hole circle (at 7.75 -9) (size 1.524 1.524) (drill 0.762) (layers "*.Cu" "*.Mask") (remove_unused_layers no) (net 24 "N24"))
  (pad "8" thru_hole circle (at 5.25 -9) (size 1.524 1.524) (drill 0.762) (layers "*.Cu" "*.Mask") (remove_unused_layers no) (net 18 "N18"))
  (pad "9" thru_hole circle (at 2.75 -9) (size 1.524 1.524) (drill 0.762) (layers "*.Cu" "*.Mask") (remove_unused_layers no) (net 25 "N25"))
  (pad "10" thru_hole circle (at 0.25 -9) (size 1.524 1.524) (drill 0.762) (layers "*.Cu" "*.Mask") (remove_unused_layers no) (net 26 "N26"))
  (pad "11" thru_hole circle (at -2.25 -9) (size 1.524 1.524) (drill 0.762) (layers "*.Cu" "*.Mask") (remove_unused_layers no)
   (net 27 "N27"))
  (pad "12" thru_hole circle (at -4.75 -9) (size 1.524 1.524) (drill 0.762) (layers "*.Cu" "*.Mask") (remove_unused_layers no)
   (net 15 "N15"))
  (pad "13" thru_hole circle (at -7.25 -9) (size 1.524 1.524) (drill 0.762) (layers "*.Cu" "*.Mask") (remove_unused_layers no)
   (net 16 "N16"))
  (pad "14" thru_hole circle (at -9.75 -9) (size 1.524 1.524) (drill 0.762) (layers "*.Cu" "*.Mask") (remove_unused_layers no)
   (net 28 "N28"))
  (pad "16" thru_hole circle (at -12.25 -9) (size 1.524 1.524) (drill 0.762) (layers "*.Cu" "*.Mask") (remove_unused_layers no)
   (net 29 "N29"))
  (pad "23" thru_hole circle (at -12.25 16.75) (size 1.524 1.524) (drill 0.762) (layers "*.Cu" "*.Mask") (remove_unused_layers no)
   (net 4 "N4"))
  (pad "24" thru_hole circle (at -9.75 16.75) (size 1.524 1.524) (drill 0.762) (layers "*.Cu" "*.Mask") (remove_unused_layers no)
   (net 5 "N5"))
  (pad "26" thru_hole circle (at -7.25 16.75) (size 1.524 1.524) (drill 0.762) (layers "*.Cu" "*.Mask") (remove_unused_layers no)
   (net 10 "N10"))
  (pad "27" thru_hole circle (at -4.75 16.75) (size 1.524 1.524) (drill 0.762) (layers "*.Cu" "*.Mask") (remove_unused_layers no)
   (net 11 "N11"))
  (pad "28" thru_hole circle (at -2.25 16.75) (size 1.524 1.524) (drill 0.762) (layers "*.Cu" "*.Mask") (remove_unused_layers no)
   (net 12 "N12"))
  (pad "29" thru_hole circle (at 0.25 16.75) (size 1.524 1.524) (drill 0.762) (layers "*.Cu" "*.Mask") (remove_unused_layers no)
   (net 13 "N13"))
  (pad "30" thru_hole circle (at 2.75 16.75) (size 1.524 1.524) (drill 0.762) (layers "*.Cu" "*.Mask") (remove_unused_layers no)
   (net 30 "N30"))
  (pad "31" thru_hole circle (at 5.25 16.75) (size 1.524 1.524) (drill 0.762) (layers "*.Cu" "*.Mask") (remove_unused_layers no)
   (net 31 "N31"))
  (pad "33" thru_hole circle (at 7.75 16.75) (size 1.524 1.524) (drill 0.762) (layers "*.Cu" "*.Mask") (remove_unused_layers no)
   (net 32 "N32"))
  (pad "34" thru_hole circle (at 10.25 16.75) (size 1.524 1.524) (drill 0.762) (layers "*.Cu" "*.Mask") (remove_unused_layers no)
   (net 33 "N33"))
  (pad "35" thru_hole circle (at 12.75 16.75) (size 1.524 1.524) (drill 0.762) (layers "*.Cu" "*.Mask") (remove_unused_layers no)
   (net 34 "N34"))
  (pad "36" thru_hole circle (at 15.25 16.75) (size 1.524 1.524) (drill 0.762) (layers "*.Cu" "*.Mask") (remove_unused_layers no)
   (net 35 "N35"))
  (pad "37" thru_hole circle (at 17.75 16.75) (size 1.524 1.524) (drill 0.762) (layers "*.Cu" "*.Mask") (remove_unused_layers no)
   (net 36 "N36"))
  (pad "38" thru_hole circle (at -14.738 16.75) (size 1.524 1.524) (drill 0.762) (layers "*.Cu" "*.Mask") (remove_unused_layers no)
   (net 1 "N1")))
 (gr_rect (start 129.5 43) (end 229 142.5) (locked yes) (stroke (width 0.05) (type default)) (fill none) (layer "Edge.Cuts"))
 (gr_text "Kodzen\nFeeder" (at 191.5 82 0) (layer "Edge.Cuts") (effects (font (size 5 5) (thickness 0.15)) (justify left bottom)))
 (segment (start 220.8383 47.5) (end 221.2983 47.96) (width 0.2) (layer "F.Cu") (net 14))
 (segment (start 183.62 47.5) (end 220.8383 47.5) (width 0.2) (layer "F.Cu") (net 14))
 (segment (start 222.5 47.96) (end 221.2983 47.96) (width 0.2) (layer "F.Cu") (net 14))
 (segment (start 216.552 56.448) (end 222.5 50.5) (width 0.2) (layer "F.Cu") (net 15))
 (segment (start 159.202 56.448) (end 216.552 56.448) (width 0.2) (layer "F.Cu") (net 15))
 (segment (start 152.5 63.15) (end 159.202 56.448) (width 0.2) (layer "F.Cu") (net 15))
 (segment (start 174.96 106.5) (end 173.7583 106.5) (width 0.2) (layer "F.Cu") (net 2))
 (segment (start 172.9119 108.1321) (end 173.7583 107.2857) (width 0.2) (layer "F.Cu") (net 2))
 (segment (start 141.94 106.5) (end 143.5721 108.1321) (width 0.2) (layer "F.Cu") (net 2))
 (segment (start 143.5721 108.1321) (end 172.9119 108.1321) (width 0.2) (layer "F.Cu") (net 2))
 (segment (start 173.7583 107.2857) (end 173.7583 106.5) (width 0.2) (layer "F.Cu") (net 2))
 (segment (start 140 88.9) (end 141.94 90.84) (width 0.2) (layer "B.Cu") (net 2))
 (segment (start 141.94 90.84) (end 141.94 106.5) (width 0.2) (layer "B.Cu") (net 2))
 (segment (start 167.34 103.74) (end 167.34 106.5) (width 0.2) (layer "B.Cu") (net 11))
 (segment (start 152.5 88.9) (end 167.34 103.74) (width 0.2) (layer "B.Cu") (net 11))
 (segment (start 133 100.81) (end 138.374 100.81) (width 0.2) (layer "F.Cu") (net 3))
 (segment (start 138.374 100.81) (end 143.2783 105.7143) (width 0.2) (layer "F.Cu") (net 3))
 (segment (start 143.2783 105.7143) (end 143.2783 106.5) (width 0.2) (layer "F.Cu") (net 3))
 (segment (start 144.48 106.5) (end 143.2783 106.5) (width 0.2) (layer "F.Cu") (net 3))
 (segment (start 138.222 93.19) (end 142.512 88.9) (width 0.2) (layer "F.Cu") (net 1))
 (segment (start 133 93.19) (end 138.222 93.19) (width 0.2) (layer "F.Cu") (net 1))
 (segment (start 176.2983 107.3262) (end 175.5228 108.1017) (width 0.2) (layer "B.Cu") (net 1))
 (segment (start 150.7617 107.2858) (end 150.7617 106.5) (width 0.2) (layer "B.Cu") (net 1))
 (segment (start 149.56 106.5) (end 148.3583 106.5) (width 0.2) (layer "B.Cu") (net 1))
 (segment (start 177.5 106.5) (end 176.2983 106.5) (width 0.2) (layer "B.Cu") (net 1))
 (segment (start 133 93.19) (end 139.4 99.59) (width 0.2) (layer "B.Cu") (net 1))
 (segment (start 140.6017 106.5) (end 140.6017 107.3262) (width 0.2) (layer "B.Cu") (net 1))
 (segment (start 149.56 106.5) (end 150.7617 106.5) (width 0.2) (layer "B.Cu") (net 1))
 (segment (start 139.4 99.59) (end 139.4 106.5) (width 0.2) (layer "B.Cu") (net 1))
 (segment (start 151.5776 108.1017) (end 150.7617 107.2858) (width 0.2) (layer "B.Cu") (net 1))
 (segment (start 147.5119 108.1321) (end 148.3583 107.2857) (width 0.2) (layer "B.Cu") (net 1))
 (segment (start 141.4076 108.1321) (end 147.5119 108.1321) (width 0.2) (layer "B.Cu") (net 1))
 (segment (start 176.2983 106.5) (end 176.2983 107.3262) (width 0.2) (layer "B.Cu") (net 1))
 (segment (start 148.3583 107.2857) (end 148.3583 106.5) (width 0.2) (layer "B.Cu") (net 1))
 (segment (start 139.4 106.5) (end 140.6017 106.5) (width 0.2) (layer "B.Cu") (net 1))
 (segment (start 175.5228 108.1017) (end 151.5776 108.1017) (width 0.2) (layer "B.Cu") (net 1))
 (segment (start 140.6017 107.3262) (end 141.4076 108.1321) (width 0.2) (layer "B.Cu") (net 1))
 (segment (start 147.02 106.5) (end 145.8183 106.5) (width 0.2) (layer "B.Cu") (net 4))
 (segment (start 145.8183 89.7183) (end 145.8183 106.5) (width 0.2) (layer "B.Cu") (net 4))
 (segment (start 145 88.9) (end 145.8183 89.7183) (width 0.2) (layer "B.Cu") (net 4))
 (segment (start 164.8 103.7) (end 164.8 106.5) (width 0.2) (layer "B.Cu") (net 10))
 (segment (start 150 88.9) (end 164.8 103.7) (width 0.2) (layer "B.Cu") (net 10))
 (segment (start 157.5 88.9) (end 172.42 103.82) (width 0.2) (layer "B.Cu") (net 13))
 (segment (start 172.42 103.82) (end 172.42 106.5) (width 0.2) (layer "B.Cu") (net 13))
 (segment (start 155 88.9) (end 169.88 103.78) (width 0.2) (layer "B.Cu") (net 12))
 (segment (start 169.88 103.78) (end 169.88 106.5) (width 0.2) (layer "B.Cu") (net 12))
 (segment (start 152.1 93.5) (end 152.1 106.5) (width 0.2) (layer "B.Cu") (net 5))
 (segment (start 147.5 88.9) (end 152.1 93.5) (width 0.2) (layer "B.Cu") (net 5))
 (segment (start 168 50) (end 168.5 49.5) (width 0.2) (layer "B.Cu") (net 18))
 (segment (start 162.5 63.15) (end 162.5 50) (width 0.2) (layer "B.Cu") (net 18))
 (segment (start 162.5 50) (end 168 50) (width 0.2) (layer "B.Cu") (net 18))
 (segment (start 162.5 50) (end 162 49.5) (width 0.2) (layer "B.Cu") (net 18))
 (segment (start 157.5 49.5) (end 149 49.5) (width 0.2) (layer "F.Cu") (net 17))
 (segment (start 168.5 45) (end 162 45) (width 0.2) (layer "F.Cu") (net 17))
 (segment (start 171 47.5) (end 174.8983 47.5) (width 0.2) (layer "F.Cu") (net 17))
 (segment (start 162 45) (end 157.5 49.5) (width 0.2) (layer "F.Cu") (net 17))
 (segment (start 168.5 45) (end 171 47.5) (width 0.2) (layer "F.Cu") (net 17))
 (segment (start 176 47.5) (end 174.8983 47.5) (width 0.2) (layer "F.Cu") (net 17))
 (segment (start 142.512 49.512) (end 142.5 49.5) (width 0.2) (layer "B.Cu") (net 17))
 (segment (start 142.512 49.512) (end 148.988 49.512) (width 0.2) (layer "B.Cu") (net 17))
 (segment (start 148.988 49.512) (end 149 49.5) (width 0.2) (layer "B.Cu") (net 17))
 (segment (start 142.512 63.15) (end 142.512 49.512) (width 0.2) (layer "B.Cu") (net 17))
 (segment (start 149 45) (end 142.5 45) (width 0.2) (layer "F.Cu") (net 16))
 (segment (start 150 63.15) (end 150.3438 62.8062) (width 0.2) (layer "B.Cu") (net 16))
 (segment (start 150.3438 46.3438) (end 149 45) (width 0.2) (layer "B.Cu") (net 16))
 (segment (start 150.3438 62.8062) (end 150.3438 46.3438) (width 0.2) (layer "B.Cu") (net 16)))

